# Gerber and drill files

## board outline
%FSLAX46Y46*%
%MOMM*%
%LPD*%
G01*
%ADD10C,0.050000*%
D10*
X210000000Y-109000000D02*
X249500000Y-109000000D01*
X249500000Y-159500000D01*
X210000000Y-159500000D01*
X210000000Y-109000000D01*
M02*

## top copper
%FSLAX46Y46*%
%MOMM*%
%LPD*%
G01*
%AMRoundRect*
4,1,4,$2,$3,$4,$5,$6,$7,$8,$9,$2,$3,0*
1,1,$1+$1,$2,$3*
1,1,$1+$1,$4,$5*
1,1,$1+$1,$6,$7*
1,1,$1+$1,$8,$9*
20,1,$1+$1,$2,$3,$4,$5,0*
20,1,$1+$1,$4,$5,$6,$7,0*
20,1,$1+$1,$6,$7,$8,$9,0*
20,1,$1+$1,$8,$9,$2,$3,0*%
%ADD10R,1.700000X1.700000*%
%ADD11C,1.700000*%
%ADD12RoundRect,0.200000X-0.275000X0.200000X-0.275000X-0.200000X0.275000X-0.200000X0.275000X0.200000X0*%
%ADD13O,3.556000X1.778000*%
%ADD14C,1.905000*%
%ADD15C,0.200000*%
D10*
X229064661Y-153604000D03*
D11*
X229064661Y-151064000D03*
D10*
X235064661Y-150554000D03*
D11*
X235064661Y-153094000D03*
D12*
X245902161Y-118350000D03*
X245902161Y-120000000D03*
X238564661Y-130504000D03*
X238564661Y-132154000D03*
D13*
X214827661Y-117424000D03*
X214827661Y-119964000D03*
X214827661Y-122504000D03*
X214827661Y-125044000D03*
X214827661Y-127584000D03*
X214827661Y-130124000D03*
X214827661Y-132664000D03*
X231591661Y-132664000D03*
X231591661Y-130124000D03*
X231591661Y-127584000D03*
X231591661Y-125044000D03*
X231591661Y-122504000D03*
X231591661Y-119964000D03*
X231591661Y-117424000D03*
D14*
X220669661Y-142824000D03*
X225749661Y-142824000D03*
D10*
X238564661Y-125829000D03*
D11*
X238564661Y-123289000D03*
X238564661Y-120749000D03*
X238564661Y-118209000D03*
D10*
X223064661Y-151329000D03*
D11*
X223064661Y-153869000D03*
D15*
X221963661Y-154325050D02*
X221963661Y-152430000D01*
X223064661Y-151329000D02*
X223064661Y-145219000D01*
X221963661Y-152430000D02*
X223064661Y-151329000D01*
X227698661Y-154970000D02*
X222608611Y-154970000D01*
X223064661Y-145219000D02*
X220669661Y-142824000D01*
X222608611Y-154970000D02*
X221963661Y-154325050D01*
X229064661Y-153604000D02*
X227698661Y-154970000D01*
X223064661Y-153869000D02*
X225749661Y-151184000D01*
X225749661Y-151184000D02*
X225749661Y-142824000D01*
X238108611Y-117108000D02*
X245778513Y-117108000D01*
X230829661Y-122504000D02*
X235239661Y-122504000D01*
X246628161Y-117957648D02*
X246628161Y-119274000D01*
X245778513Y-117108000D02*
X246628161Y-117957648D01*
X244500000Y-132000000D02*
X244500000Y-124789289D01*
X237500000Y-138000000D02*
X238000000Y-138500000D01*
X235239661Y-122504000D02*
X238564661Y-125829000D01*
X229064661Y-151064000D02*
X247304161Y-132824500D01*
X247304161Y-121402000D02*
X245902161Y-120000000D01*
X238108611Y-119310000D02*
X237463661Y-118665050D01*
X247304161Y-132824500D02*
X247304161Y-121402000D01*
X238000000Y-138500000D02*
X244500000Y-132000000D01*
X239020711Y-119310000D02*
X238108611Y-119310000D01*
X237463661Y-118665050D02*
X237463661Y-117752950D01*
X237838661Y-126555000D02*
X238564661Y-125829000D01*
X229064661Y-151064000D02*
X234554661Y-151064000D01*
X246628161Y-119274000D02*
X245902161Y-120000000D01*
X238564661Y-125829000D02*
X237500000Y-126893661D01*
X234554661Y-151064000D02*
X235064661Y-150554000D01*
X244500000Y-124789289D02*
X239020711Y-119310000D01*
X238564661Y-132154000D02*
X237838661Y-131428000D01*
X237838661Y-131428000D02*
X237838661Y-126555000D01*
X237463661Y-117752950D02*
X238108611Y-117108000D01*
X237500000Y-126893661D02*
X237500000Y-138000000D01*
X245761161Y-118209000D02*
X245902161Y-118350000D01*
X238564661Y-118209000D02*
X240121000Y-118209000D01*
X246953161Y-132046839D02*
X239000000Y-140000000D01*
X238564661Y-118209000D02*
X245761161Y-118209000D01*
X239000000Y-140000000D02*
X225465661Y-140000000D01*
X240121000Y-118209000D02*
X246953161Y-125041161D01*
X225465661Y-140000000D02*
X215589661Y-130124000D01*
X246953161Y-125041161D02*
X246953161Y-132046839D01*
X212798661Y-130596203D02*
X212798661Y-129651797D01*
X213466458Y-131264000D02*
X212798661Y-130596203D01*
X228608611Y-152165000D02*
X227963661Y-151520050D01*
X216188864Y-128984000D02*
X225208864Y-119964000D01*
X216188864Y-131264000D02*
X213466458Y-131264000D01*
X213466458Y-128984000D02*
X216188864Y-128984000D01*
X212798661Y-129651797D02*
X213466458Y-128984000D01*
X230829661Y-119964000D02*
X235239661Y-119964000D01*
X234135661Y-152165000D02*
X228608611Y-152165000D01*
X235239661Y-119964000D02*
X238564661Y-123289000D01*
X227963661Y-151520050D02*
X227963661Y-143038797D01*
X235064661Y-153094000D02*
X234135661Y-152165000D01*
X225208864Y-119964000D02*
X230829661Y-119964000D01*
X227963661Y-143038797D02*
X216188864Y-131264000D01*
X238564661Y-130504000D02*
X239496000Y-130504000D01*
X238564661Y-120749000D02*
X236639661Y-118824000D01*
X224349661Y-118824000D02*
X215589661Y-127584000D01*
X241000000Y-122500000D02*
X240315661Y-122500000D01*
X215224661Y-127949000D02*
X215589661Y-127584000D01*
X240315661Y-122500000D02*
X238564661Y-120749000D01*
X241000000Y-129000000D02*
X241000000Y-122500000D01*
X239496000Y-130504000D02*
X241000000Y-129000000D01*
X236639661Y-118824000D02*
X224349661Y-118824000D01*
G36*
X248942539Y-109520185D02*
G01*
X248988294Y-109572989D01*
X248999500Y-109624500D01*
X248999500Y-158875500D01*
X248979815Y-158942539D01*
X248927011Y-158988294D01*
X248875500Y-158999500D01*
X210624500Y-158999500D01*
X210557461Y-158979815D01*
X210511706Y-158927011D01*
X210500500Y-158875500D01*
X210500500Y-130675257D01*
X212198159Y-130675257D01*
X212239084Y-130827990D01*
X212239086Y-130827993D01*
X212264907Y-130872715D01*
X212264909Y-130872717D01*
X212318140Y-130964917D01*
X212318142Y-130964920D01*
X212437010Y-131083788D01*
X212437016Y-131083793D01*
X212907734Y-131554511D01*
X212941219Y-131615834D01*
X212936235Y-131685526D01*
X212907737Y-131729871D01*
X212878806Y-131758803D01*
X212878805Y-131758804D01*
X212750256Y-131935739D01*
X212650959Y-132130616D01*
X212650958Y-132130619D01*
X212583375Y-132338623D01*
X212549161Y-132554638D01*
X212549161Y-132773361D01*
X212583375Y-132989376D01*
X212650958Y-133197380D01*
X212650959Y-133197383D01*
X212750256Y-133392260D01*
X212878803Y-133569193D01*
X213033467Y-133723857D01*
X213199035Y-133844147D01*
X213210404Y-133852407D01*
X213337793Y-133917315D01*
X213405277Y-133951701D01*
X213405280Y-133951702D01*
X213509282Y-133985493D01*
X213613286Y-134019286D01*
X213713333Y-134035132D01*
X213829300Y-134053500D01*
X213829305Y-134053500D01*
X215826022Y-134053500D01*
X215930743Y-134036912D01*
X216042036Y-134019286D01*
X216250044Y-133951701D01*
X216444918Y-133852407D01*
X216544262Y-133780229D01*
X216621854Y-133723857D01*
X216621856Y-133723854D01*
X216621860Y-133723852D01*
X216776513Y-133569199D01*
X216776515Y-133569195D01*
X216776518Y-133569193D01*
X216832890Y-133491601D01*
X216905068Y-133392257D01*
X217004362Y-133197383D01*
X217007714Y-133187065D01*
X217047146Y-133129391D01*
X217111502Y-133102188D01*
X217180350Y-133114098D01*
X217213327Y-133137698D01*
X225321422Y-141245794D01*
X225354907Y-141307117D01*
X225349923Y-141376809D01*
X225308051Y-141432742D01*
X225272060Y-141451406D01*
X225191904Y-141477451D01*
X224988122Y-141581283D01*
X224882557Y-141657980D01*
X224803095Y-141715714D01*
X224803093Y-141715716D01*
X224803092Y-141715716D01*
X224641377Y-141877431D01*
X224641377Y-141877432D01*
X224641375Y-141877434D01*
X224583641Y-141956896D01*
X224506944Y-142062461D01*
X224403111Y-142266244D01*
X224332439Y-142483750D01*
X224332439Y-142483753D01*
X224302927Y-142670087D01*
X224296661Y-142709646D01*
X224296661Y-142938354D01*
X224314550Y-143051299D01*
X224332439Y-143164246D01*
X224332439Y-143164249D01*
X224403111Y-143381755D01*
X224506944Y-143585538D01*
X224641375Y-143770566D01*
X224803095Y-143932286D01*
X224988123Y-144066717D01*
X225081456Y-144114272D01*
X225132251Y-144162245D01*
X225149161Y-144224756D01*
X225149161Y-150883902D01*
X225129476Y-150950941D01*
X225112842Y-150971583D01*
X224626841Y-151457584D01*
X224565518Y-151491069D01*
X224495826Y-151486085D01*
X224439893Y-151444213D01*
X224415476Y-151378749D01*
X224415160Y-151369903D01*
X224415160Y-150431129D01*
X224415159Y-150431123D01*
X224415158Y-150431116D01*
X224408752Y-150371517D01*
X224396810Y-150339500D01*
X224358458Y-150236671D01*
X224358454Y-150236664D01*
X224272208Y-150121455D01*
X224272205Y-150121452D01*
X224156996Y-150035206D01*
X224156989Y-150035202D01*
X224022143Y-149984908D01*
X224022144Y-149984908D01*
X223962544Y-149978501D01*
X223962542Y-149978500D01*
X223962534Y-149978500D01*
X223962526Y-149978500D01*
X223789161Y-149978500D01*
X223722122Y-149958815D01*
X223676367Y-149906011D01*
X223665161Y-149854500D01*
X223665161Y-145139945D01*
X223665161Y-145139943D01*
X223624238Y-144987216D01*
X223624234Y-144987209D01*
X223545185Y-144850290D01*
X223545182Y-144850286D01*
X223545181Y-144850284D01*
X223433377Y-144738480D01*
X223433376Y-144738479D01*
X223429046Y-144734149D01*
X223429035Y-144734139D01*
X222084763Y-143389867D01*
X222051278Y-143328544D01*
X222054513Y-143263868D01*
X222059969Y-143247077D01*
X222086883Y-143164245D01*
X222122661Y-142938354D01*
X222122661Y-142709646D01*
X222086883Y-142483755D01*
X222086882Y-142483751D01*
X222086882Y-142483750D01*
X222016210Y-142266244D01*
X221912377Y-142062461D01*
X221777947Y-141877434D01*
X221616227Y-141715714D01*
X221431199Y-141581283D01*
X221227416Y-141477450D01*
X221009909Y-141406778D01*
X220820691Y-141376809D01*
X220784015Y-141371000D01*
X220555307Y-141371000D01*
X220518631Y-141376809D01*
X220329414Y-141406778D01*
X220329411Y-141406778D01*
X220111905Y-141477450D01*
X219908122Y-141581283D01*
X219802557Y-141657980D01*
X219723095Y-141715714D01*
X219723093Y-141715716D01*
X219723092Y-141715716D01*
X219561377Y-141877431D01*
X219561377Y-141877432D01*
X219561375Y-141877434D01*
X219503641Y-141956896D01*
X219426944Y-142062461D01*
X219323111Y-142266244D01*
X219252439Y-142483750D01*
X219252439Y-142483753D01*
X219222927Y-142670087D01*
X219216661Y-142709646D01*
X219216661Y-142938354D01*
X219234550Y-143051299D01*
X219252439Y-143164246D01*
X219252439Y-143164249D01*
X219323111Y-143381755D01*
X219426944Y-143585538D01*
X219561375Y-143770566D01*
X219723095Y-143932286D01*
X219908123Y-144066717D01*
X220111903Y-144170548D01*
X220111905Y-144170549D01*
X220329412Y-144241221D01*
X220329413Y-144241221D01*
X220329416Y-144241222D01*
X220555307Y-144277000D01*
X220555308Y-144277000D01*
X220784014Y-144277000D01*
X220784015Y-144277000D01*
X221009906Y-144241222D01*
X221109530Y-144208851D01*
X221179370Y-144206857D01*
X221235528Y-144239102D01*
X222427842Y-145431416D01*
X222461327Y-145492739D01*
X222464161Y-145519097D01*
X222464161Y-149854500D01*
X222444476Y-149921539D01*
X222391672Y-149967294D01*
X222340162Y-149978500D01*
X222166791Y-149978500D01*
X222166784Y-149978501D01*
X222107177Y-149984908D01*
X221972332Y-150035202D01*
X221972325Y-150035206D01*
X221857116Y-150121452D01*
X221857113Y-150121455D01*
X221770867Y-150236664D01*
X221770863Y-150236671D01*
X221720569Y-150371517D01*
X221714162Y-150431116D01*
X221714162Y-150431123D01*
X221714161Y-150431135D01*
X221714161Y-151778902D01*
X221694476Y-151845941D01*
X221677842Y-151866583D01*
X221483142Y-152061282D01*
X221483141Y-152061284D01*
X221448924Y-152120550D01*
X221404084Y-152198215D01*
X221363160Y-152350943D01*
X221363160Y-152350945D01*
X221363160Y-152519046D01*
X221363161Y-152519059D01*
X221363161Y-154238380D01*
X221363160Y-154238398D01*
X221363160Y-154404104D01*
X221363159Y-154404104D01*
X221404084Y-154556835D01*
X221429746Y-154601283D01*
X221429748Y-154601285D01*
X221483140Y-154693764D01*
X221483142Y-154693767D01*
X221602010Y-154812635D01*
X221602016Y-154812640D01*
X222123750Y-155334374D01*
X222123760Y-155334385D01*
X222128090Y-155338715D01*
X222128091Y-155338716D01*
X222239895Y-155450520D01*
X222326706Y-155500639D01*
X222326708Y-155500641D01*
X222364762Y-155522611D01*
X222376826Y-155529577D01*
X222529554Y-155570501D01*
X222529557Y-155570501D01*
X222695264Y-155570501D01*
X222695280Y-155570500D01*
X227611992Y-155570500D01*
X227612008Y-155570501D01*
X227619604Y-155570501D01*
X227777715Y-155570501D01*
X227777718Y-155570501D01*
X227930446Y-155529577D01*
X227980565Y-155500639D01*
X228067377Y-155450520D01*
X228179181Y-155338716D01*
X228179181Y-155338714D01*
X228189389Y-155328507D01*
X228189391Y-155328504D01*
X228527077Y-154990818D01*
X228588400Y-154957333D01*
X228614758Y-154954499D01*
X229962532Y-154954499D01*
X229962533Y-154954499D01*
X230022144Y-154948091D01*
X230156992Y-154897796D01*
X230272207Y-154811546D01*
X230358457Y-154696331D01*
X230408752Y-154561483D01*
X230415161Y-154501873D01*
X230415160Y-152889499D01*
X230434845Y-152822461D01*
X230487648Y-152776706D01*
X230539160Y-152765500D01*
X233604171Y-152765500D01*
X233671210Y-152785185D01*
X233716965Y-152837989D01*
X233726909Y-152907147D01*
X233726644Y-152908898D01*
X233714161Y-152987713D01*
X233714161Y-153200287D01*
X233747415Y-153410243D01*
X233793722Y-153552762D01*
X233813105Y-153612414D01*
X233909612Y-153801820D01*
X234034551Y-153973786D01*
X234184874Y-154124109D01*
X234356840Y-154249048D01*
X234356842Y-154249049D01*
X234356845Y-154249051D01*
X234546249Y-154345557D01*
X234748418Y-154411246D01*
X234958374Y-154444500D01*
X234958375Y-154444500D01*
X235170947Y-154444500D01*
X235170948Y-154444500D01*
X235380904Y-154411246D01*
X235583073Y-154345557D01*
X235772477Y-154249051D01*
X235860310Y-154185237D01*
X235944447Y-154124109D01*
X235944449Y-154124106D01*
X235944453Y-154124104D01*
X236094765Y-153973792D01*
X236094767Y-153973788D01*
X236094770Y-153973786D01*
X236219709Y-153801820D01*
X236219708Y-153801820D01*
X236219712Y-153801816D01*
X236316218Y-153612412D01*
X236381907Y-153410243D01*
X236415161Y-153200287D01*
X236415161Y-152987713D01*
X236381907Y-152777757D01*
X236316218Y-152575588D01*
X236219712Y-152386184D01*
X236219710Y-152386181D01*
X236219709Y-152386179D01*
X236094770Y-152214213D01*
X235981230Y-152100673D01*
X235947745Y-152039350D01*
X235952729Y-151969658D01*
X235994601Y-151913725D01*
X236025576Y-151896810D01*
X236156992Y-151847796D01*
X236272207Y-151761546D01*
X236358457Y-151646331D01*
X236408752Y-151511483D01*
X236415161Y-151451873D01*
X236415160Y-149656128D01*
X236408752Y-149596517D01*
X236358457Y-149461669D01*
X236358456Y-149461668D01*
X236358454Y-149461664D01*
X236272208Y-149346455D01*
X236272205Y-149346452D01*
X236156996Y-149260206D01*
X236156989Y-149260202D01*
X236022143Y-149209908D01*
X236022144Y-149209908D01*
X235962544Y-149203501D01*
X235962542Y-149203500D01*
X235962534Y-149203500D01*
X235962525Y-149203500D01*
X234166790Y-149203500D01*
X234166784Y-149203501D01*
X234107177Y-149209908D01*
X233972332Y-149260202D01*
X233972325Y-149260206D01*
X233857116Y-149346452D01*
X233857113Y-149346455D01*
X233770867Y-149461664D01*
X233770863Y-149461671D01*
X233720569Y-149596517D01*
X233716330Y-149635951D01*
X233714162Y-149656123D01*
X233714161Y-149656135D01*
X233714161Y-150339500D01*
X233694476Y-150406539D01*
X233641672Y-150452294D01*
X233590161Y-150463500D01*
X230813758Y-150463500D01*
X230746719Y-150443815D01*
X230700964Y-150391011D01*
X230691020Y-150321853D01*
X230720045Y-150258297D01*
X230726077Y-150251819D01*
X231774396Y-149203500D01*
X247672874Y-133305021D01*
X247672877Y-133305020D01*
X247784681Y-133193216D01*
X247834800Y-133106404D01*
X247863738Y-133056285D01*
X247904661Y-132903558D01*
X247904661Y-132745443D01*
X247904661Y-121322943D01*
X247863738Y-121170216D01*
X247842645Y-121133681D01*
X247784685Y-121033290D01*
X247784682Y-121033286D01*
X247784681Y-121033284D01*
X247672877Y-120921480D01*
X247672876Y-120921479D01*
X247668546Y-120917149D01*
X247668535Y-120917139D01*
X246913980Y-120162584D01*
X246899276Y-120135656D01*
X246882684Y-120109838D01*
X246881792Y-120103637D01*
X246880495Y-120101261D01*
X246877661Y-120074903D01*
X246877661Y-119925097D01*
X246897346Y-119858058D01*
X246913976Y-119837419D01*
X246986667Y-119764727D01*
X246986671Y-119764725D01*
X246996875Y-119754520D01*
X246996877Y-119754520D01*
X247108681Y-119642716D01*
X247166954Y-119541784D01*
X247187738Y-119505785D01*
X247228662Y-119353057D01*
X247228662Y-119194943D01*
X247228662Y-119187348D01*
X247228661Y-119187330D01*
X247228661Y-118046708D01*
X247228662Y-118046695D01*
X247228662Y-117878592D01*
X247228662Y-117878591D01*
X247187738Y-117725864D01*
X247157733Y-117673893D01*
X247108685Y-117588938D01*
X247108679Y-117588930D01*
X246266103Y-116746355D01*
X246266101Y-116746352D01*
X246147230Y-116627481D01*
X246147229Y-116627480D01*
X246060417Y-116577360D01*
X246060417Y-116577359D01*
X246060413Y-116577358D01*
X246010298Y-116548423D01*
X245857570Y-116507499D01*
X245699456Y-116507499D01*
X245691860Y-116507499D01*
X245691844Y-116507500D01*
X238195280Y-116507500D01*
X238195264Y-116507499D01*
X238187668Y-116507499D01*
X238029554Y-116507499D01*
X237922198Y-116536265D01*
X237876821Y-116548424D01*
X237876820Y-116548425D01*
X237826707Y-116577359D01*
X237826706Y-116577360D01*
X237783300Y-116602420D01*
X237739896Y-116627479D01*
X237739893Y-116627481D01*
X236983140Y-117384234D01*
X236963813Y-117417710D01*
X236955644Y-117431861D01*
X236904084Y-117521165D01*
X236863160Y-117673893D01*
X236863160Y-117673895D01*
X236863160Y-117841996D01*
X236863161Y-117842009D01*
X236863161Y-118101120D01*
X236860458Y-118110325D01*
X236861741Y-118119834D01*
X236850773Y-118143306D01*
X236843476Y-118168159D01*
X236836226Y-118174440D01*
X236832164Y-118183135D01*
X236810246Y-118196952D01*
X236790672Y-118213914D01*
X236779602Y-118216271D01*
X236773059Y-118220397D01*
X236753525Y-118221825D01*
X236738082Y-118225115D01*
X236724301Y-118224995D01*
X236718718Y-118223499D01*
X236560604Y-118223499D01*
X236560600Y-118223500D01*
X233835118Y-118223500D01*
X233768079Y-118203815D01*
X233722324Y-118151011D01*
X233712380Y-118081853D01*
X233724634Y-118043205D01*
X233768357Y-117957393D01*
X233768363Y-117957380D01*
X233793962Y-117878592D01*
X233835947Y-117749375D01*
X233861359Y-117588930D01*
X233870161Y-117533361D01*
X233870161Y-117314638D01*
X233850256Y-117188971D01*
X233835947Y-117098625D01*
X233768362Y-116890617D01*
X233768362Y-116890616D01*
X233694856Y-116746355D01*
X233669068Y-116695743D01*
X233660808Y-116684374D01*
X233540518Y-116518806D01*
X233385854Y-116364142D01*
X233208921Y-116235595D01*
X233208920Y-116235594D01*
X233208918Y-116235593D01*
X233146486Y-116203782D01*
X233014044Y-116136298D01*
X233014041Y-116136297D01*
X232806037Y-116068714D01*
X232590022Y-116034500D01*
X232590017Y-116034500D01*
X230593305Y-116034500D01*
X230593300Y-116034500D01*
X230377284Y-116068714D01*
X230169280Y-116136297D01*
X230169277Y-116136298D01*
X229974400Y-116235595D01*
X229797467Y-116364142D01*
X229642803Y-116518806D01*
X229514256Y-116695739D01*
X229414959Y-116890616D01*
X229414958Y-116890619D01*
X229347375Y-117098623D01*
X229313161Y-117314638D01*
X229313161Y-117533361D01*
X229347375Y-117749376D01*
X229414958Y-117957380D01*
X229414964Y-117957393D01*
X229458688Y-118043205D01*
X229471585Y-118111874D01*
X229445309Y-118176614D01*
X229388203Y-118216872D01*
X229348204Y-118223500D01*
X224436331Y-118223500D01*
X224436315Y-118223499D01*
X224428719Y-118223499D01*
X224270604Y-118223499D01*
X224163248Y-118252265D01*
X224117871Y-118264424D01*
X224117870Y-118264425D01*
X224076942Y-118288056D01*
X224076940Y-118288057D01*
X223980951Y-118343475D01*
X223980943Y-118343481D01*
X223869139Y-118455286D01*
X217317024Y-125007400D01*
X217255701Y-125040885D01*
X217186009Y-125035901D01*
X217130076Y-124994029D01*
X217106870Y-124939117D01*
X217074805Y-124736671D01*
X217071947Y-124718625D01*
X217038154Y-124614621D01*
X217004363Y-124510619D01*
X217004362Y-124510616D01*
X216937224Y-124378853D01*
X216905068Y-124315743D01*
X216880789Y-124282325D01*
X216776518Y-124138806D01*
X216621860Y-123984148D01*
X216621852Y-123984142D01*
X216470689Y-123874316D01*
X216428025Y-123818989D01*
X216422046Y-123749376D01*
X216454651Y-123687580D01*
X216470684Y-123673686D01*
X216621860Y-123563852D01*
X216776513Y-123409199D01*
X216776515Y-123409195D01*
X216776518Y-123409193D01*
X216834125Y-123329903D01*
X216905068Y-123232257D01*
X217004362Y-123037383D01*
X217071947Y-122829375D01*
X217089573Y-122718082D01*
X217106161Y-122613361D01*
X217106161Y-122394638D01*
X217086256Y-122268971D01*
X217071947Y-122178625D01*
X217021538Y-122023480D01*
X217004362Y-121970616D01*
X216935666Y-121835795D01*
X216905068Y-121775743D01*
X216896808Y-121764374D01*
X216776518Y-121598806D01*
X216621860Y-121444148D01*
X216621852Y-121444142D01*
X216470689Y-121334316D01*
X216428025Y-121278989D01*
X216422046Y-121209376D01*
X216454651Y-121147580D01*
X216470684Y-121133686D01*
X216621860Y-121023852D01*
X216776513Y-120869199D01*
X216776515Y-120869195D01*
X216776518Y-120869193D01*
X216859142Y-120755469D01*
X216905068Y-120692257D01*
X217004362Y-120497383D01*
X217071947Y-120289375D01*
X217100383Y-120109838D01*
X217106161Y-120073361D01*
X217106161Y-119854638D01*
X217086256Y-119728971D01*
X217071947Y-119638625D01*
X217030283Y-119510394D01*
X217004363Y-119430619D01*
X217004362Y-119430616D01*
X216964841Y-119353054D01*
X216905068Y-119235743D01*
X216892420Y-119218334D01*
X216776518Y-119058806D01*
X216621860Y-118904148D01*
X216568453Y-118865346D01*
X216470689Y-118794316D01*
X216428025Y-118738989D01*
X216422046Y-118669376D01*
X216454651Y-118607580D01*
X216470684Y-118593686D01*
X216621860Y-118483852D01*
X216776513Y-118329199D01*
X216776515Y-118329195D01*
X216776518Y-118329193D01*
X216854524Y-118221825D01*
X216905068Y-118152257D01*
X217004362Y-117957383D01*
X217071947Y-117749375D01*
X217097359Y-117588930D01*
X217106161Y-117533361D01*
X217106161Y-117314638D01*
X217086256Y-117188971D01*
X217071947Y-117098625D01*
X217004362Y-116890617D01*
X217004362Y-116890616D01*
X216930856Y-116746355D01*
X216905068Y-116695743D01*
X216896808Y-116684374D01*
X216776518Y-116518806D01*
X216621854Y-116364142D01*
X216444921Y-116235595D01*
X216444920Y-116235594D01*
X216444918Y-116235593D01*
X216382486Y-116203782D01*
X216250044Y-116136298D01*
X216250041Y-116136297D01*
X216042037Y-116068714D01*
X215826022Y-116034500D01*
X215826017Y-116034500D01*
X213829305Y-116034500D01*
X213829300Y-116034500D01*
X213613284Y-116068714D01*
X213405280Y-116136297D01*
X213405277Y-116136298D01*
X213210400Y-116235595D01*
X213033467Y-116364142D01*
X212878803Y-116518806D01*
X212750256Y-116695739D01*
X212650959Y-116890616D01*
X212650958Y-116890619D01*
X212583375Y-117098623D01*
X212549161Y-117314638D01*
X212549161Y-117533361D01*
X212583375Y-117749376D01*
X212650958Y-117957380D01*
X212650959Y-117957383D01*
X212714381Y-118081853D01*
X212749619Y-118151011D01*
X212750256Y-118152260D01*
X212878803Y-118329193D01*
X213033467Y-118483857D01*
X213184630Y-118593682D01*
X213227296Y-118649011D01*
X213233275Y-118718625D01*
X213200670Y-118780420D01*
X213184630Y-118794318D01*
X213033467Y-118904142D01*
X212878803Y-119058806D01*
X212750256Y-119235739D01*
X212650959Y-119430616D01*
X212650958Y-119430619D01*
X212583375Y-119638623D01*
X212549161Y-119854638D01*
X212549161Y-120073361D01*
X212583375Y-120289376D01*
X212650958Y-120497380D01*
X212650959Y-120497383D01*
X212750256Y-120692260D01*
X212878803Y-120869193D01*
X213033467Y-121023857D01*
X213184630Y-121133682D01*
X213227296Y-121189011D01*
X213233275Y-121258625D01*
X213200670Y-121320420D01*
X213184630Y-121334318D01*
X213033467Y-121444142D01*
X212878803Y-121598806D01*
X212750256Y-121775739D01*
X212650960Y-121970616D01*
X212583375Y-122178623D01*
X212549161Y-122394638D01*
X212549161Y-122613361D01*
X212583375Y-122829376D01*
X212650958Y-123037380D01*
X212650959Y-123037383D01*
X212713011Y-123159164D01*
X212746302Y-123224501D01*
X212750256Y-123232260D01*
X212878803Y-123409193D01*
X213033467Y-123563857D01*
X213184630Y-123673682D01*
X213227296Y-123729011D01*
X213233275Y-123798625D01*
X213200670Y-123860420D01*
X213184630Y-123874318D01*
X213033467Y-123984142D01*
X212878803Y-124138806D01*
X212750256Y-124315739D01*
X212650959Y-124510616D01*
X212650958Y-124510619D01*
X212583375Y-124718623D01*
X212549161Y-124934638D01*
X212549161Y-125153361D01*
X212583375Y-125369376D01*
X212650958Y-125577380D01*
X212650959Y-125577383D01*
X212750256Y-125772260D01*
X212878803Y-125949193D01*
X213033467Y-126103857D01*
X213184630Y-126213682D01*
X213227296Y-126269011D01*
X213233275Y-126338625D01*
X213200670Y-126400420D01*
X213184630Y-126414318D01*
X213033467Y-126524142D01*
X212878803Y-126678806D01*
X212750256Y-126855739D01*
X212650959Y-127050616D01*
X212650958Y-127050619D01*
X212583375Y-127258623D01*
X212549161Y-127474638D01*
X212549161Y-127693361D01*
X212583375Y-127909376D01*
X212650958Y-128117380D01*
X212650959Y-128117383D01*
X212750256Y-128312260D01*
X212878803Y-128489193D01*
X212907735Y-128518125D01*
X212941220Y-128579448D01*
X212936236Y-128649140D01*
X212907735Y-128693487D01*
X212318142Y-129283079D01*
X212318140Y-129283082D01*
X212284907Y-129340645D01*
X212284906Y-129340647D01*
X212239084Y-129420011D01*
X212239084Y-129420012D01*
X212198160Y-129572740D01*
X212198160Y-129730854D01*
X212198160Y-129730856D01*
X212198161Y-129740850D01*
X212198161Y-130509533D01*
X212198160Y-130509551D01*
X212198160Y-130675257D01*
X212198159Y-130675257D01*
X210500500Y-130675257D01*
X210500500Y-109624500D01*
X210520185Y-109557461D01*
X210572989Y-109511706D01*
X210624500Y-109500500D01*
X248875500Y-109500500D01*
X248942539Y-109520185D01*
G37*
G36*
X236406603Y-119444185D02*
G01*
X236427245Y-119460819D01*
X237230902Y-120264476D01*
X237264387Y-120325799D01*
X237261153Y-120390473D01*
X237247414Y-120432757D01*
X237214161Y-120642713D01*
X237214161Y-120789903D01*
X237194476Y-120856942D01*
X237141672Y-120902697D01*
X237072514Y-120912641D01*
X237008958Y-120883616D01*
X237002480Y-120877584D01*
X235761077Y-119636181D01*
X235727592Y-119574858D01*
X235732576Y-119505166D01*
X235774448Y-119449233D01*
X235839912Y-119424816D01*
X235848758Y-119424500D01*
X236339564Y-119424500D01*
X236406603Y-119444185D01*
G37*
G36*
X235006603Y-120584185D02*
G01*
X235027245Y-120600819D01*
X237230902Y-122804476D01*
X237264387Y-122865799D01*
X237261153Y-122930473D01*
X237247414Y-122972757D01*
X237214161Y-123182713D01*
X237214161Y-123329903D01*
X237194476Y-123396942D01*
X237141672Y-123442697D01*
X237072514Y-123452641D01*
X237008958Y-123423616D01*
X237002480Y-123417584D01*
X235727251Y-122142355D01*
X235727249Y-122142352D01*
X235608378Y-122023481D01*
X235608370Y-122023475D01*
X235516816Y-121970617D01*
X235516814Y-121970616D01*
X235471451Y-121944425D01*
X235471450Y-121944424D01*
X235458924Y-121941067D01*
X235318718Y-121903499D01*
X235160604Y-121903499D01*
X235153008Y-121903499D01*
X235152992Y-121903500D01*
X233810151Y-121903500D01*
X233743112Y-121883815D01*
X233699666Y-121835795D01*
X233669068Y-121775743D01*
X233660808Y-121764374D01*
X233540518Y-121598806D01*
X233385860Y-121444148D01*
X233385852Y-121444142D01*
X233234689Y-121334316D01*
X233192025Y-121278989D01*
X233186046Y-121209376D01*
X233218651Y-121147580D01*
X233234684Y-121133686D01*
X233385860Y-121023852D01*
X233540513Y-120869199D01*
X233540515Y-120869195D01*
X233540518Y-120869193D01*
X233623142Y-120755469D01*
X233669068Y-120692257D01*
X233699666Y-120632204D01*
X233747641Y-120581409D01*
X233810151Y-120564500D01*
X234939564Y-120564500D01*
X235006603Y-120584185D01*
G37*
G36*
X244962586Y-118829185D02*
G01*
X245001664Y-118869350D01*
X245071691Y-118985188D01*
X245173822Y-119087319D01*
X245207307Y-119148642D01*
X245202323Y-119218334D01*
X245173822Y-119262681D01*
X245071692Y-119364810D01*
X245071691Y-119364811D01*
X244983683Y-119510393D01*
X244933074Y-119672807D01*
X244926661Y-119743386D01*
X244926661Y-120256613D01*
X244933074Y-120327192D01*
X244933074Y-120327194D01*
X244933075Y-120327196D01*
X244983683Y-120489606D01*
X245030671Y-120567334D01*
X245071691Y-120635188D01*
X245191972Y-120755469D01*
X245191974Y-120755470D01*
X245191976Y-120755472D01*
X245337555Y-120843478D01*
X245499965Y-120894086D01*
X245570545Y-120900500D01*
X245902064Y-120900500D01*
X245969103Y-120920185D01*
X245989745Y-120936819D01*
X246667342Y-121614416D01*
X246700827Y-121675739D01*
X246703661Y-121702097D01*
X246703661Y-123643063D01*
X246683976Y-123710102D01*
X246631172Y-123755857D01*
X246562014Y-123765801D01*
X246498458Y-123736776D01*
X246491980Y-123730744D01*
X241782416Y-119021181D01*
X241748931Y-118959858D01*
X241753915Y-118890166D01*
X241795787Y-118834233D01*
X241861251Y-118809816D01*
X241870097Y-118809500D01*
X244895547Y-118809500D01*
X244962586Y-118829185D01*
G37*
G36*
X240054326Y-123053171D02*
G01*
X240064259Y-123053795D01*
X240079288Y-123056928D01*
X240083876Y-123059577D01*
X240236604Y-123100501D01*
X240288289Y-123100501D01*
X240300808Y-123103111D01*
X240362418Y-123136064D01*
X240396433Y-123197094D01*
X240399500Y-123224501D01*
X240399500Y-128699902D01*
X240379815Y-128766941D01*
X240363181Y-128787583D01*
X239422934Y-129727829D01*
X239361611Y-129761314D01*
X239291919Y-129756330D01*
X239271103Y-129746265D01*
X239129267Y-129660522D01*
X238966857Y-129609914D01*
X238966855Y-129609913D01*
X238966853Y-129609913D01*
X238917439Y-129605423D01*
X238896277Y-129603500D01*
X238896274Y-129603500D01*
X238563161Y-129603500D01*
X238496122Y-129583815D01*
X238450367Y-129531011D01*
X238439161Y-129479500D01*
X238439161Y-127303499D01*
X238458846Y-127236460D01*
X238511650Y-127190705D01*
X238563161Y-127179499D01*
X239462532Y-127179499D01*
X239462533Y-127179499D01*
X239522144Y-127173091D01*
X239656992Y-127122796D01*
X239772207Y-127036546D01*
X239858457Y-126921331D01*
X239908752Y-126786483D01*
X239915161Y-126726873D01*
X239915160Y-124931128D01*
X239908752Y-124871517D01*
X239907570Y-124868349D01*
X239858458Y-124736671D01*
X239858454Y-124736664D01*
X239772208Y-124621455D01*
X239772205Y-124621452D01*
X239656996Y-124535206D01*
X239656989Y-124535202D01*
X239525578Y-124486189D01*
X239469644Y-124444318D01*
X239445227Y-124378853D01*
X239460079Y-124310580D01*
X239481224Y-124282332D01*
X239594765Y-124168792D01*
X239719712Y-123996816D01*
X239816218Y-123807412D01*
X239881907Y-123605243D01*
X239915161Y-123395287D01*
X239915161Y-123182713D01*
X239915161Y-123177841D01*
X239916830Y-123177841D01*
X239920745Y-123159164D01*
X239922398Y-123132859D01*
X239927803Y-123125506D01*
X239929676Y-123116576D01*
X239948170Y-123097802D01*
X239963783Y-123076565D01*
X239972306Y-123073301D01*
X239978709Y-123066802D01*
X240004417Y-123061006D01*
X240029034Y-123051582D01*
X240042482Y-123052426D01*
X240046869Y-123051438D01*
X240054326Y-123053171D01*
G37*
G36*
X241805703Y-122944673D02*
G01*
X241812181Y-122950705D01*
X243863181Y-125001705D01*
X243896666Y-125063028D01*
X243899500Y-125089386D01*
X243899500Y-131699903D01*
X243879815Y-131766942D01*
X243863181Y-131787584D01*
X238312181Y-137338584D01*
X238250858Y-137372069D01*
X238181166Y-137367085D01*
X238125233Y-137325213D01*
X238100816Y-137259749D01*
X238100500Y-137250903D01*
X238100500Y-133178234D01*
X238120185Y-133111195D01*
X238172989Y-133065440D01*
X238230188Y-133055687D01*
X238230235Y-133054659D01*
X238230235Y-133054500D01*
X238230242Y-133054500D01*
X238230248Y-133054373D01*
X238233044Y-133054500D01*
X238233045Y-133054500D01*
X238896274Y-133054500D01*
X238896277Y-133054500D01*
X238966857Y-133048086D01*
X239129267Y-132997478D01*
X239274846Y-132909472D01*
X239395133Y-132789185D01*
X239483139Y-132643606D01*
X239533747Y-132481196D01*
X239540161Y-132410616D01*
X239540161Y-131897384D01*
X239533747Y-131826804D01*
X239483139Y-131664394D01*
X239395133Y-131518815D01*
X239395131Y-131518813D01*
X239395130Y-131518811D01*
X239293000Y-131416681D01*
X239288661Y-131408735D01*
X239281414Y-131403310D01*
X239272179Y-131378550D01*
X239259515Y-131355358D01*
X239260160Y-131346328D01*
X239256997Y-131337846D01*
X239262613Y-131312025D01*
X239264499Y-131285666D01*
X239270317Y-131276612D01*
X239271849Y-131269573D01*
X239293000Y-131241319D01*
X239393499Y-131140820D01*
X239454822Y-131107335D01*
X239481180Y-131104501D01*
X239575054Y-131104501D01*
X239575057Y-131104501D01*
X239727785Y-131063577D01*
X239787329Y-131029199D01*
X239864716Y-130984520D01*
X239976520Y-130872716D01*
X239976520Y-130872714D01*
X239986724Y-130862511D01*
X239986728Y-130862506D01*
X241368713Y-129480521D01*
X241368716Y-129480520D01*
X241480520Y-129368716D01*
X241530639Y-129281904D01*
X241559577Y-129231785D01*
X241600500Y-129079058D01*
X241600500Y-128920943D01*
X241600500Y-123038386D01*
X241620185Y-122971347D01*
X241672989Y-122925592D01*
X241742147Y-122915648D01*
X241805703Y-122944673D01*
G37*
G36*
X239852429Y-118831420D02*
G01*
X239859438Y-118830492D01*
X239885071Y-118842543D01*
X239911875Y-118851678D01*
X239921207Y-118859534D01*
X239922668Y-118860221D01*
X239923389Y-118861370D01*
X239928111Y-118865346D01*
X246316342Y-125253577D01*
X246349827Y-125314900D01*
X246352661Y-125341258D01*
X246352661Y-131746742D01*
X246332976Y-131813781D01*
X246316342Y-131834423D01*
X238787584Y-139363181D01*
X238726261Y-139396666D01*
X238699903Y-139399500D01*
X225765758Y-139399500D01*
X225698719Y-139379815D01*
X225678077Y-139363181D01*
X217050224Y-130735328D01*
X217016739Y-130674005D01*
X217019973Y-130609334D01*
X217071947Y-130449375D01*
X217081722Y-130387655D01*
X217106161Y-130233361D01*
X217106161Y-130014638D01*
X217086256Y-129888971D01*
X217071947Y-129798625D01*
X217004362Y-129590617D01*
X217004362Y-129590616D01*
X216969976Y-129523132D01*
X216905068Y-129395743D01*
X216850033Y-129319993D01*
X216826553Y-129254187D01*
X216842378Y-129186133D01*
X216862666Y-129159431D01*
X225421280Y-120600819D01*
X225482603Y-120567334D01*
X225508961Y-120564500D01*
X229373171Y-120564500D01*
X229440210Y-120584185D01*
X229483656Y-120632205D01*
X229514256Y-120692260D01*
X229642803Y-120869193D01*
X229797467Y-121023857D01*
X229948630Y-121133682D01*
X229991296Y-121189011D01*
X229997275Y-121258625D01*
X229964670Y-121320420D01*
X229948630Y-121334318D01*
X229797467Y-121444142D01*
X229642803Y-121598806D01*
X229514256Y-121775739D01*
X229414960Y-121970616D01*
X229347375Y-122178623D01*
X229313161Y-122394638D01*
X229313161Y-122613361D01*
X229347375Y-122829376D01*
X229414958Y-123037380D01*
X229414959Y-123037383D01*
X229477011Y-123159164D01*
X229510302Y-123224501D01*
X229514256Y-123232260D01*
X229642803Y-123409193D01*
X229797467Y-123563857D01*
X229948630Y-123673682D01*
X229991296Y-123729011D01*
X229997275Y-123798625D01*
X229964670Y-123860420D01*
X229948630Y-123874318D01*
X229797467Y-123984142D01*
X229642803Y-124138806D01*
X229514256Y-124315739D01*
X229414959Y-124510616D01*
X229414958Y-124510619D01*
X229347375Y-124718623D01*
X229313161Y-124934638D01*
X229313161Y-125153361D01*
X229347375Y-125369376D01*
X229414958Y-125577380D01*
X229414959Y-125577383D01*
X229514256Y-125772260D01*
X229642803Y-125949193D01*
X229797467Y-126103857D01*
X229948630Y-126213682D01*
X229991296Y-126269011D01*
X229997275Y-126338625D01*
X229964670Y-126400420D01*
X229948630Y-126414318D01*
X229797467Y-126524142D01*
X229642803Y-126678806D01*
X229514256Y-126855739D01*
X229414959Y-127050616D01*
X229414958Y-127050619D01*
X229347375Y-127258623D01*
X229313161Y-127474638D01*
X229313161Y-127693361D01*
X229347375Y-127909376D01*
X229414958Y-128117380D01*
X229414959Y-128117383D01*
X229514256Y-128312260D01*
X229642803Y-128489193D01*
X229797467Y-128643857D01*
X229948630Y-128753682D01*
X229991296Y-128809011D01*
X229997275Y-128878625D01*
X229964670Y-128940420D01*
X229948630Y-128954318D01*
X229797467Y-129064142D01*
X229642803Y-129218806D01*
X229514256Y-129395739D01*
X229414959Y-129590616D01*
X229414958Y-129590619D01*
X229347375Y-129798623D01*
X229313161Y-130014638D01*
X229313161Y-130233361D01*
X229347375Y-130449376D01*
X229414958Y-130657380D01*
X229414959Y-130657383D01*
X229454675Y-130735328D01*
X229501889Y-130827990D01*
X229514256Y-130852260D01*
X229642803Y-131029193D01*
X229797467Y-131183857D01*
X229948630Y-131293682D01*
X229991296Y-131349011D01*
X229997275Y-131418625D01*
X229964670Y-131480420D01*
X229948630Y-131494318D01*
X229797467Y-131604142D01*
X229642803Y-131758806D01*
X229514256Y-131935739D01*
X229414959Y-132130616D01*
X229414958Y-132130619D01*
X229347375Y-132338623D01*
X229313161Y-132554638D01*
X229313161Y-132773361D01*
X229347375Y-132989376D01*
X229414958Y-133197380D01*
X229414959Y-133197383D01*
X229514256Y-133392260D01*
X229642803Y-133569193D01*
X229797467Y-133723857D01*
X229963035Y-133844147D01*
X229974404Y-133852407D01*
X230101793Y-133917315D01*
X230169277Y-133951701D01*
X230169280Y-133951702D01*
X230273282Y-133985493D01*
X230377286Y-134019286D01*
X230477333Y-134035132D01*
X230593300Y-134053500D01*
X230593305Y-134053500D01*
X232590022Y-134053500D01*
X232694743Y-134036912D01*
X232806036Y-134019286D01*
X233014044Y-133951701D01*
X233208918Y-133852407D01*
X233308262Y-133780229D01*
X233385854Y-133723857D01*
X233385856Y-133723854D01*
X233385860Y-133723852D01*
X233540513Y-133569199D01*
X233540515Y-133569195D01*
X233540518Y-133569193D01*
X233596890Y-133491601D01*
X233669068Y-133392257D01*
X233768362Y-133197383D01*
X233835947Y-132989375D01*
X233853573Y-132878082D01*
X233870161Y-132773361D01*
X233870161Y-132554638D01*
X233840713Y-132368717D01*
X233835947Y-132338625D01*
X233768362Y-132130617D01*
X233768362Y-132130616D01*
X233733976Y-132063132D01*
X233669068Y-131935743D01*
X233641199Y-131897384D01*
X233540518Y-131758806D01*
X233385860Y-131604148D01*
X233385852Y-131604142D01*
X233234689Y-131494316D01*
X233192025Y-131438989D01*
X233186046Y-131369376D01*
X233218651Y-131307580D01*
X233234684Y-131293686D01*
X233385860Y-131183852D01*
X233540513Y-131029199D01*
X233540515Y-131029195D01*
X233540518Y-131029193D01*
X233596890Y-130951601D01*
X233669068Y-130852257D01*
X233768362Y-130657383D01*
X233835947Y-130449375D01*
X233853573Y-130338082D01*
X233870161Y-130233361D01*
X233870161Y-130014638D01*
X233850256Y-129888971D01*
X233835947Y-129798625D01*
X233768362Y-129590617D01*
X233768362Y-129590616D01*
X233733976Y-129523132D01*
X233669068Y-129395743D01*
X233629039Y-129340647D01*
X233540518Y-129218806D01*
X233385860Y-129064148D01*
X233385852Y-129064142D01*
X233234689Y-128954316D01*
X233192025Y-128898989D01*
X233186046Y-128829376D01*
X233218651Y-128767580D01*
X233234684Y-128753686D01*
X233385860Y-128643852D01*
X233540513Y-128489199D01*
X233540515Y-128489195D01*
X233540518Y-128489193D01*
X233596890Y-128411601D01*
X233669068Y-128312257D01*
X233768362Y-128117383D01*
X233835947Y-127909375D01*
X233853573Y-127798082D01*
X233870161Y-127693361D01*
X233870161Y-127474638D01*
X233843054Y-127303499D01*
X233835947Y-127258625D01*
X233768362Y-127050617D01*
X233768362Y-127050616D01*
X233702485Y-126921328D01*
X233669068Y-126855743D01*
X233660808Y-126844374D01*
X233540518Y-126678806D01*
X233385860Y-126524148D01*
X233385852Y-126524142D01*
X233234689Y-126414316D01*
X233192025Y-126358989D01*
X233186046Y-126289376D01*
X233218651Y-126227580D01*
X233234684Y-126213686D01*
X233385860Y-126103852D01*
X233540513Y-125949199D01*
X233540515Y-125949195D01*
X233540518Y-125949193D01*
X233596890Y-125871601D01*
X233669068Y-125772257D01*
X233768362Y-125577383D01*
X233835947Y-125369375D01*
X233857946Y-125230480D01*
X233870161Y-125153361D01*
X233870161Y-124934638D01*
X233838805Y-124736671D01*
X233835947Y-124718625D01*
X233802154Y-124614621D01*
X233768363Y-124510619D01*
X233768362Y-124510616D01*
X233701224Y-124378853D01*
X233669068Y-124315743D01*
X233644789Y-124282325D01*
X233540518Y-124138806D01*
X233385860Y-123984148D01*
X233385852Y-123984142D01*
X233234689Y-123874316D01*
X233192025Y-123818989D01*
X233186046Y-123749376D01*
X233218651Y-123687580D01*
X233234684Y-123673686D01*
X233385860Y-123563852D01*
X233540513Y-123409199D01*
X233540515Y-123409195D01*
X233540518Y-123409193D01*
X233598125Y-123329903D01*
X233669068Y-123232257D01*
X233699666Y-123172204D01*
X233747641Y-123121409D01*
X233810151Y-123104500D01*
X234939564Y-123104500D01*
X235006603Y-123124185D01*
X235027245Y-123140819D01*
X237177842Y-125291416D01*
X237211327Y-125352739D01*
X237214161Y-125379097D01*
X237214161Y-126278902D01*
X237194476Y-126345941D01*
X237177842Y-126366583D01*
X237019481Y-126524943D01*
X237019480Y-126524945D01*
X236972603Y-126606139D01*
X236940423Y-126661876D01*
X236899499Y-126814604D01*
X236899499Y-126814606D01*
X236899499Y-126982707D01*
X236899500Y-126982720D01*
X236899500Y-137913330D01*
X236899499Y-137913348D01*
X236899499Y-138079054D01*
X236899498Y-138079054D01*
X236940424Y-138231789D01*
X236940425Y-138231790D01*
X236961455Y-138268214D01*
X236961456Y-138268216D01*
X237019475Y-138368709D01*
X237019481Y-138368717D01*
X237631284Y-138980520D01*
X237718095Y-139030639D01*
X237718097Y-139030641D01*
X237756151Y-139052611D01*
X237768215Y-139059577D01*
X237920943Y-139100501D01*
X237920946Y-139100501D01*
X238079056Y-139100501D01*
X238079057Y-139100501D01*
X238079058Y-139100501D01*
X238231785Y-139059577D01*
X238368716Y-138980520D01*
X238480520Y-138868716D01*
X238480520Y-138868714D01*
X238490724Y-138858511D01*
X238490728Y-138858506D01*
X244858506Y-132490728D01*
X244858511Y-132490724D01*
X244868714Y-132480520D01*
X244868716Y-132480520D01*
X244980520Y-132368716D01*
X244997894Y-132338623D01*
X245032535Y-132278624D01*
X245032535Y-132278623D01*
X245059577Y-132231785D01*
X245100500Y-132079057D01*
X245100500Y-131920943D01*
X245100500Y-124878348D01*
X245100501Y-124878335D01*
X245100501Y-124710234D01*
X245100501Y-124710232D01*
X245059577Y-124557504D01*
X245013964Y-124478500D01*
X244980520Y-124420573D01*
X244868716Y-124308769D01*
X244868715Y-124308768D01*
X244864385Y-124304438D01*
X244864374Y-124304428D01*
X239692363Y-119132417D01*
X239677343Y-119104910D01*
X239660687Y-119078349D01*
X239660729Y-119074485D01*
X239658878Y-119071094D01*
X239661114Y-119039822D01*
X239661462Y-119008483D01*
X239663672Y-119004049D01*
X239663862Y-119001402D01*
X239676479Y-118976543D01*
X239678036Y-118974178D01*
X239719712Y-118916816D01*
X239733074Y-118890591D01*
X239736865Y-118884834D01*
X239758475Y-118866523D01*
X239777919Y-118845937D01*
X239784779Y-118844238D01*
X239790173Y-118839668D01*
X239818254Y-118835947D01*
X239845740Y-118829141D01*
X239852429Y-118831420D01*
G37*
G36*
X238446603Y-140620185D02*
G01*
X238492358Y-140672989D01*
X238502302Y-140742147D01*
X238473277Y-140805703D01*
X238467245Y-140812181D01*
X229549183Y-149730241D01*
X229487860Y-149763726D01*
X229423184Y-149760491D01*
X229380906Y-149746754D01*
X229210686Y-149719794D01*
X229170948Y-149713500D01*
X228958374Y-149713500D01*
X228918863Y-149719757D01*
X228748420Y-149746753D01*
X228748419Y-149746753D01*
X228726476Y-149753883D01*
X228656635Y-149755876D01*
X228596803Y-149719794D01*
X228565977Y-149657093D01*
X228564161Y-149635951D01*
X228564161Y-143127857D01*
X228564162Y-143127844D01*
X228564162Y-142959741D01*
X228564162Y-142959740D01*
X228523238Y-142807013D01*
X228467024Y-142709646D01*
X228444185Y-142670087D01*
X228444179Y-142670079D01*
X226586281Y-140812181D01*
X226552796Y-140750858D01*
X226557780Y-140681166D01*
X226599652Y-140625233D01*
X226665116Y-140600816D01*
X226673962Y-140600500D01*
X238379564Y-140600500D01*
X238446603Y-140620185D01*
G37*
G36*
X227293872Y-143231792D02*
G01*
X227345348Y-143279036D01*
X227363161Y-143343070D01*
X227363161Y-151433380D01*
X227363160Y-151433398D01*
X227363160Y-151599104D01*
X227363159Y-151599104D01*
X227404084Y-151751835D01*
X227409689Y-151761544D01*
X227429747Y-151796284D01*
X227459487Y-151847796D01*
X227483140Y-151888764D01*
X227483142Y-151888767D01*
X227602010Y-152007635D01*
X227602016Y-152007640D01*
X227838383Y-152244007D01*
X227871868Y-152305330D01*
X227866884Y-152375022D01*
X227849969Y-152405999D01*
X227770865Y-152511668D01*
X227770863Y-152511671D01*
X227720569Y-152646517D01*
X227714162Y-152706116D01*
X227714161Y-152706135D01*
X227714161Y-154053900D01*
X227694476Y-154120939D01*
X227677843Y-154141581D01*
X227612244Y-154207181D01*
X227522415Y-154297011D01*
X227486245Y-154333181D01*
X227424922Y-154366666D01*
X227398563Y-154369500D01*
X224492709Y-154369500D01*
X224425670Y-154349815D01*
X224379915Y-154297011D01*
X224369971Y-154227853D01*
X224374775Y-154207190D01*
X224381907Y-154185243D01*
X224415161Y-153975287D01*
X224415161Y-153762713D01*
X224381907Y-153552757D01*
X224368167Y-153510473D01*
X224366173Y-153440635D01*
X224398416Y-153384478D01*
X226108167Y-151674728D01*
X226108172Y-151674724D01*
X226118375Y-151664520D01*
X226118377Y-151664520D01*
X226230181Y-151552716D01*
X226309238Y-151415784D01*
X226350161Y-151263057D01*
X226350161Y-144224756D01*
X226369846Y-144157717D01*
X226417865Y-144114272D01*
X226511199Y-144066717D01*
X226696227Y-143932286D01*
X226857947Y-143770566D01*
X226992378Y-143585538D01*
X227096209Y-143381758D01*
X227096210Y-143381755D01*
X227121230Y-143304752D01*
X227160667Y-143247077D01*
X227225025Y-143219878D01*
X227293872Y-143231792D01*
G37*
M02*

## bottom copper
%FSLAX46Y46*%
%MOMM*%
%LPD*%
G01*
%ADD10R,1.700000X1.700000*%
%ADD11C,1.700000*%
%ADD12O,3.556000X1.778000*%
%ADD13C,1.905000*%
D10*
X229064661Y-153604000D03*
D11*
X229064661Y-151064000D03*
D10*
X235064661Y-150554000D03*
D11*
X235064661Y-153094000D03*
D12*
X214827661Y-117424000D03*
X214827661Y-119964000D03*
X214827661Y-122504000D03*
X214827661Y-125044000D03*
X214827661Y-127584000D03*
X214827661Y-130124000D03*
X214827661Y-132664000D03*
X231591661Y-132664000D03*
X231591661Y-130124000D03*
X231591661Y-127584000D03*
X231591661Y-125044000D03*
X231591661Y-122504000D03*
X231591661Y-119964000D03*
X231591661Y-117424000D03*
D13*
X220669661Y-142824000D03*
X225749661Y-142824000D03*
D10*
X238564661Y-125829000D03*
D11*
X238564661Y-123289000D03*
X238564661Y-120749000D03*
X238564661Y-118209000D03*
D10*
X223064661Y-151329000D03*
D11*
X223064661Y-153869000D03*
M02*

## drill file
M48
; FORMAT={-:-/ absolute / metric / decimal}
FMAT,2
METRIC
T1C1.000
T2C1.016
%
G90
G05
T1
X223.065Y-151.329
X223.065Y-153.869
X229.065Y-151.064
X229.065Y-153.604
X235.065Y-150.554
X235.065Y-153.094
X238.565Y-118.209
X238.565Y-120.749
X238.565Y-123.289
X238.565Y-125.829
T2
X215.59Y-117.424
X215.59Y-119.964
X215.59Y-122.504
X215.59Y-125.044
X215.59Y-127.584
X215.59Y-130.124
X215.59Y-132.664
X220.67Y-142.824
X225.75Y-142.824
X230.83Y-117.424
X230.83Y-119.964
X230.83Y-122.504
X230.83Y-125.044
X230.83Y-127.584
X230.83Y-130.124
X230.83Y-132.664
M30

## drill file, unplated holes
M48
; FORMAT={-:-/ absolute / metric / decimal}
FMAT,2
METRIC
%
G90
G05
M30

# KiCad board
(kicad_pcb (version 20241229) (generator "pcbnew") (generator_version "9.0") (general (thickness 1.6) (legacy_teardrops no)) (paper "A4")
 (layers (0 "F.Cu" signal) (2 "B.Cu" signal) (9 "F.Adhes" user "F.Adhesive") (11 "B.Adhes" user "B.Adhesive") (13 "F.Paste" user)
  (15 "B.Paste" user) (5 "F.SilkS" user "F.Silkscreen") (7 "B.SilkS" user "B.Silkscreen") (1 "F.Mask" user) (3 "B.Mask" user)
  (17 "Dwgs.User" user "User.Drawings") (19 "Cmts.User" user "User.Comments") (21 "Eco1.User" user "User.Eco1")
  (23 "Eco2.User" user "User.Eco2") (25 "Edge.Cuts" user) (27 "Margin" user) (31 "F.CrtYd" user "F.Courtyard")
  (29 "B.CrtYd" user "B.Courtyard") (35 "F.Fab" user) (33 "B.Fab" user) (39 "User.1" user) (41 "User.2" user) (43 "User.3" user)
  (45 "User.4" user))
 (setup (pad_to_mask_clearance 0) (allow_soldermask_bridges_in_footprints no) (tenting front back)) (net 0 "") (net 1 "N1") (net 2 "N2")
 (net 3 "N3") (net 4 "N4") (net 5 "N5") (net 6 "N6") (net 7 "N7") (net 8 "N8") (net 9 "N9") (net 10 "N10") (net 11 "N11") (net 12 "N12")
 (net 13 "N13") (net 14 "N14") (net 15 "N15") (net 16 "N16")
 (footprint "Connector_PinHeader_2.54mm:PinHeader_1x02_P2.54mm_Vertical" (layer "F.Cu") (at 229.064661 153.604 180)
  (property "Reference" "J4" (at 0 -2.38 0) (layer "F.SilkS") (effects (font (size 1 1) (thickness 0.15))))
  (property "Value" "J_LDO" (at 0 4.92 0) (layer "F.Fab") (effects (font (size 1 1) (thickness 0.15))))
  (pad "1" thru_hole rect (at 0 0 180) (size 1.7 1.7) (drill 1) (layers "*.Cu" "*.Mask") (remove_unused_layers no) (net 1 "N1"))
  (pad "2" thru_hole circle (at 0 2.54 180) (size 1.7 1.7) (drill 1) (layers "*.Cu" "*.Mask") (remove_unused_layers no) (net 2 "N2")))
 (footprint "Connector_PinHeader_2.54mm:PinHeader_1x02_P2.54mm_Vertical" (layer "F.Cu") (at 235.064661 150.554)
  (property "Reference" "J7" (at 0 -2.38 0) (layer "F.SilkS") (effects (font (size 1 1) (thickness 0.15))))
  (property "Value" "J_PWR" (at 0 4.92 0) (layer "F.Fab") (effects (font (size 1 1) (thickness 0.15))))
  (pad "1" thru_hole rect (at 0 0) (size 1.7 1.7) (drill 1) (layers "*.Cu" "*.Mask") (remove_unused_layers no) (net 2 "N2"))
  (pad "2" thru_hole circle (at 0 2.54) (size 1.7 1.7) (drill 1) (layers "*.Cu" "*.Mask") (remove_unused_layers no) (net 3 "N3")))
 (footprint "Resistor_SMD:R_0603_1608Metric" (layer "F.Cu") (at 245.902161 119.175 -90)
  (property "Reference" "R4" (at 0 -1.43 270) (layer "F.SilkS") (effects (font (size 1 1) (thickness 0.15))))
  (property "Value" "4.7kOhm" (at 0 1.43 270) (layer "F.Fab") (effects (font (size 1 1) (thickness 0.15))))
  (pad "1" smd roundrect (at -0.825 0 270) (size 0.8 0.95) (layers "F.Cu" "F.Mask" "F.Paste") (roundrect_rratio 0.25) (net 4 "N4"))
  (pad "2" smd roundrect (at 0.825 0 270) (size 0.8 0.95) (layers "F.Cu" "F.Mask" "F.Paste") (roundrect_rratio 0.25) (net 2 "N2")))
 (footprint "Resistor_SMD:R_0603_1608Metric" (layer "F.Cu") (at 238.564661 131.329 -90)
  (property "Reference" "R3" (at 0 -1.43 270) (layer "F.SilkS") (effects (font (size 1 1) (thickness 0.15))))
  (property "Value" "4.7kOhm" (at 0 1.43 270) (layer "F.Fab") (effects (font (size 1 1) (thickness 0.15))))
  (pad "1" smd roundrect (at -0.825 0 270) (size 0.8 0.95) (layers "F.Cu" "F.Mask" "F.Paste") (roundrect_rratio 0.25) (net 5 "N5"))
  (pad "2" smd roundrect (at 0.825 0 270) (size 0.8 0.95) (layers "F.Cu" "F.Mask" "F.Paste") (roundrect_rratio 0.25) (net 2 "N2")))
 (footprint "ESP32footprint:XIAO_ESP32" (layer "F.Cu") (at 223.209661 125.044)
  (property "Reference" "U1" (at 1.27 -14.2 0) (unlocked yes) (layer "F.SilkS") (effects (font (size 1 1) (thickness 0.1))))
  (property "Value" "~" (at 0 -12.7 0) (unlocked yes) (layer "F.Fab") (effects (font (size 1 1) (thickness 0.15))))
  (pad "1" thru_hole oval (at -7.62 -7.62) (size 3.556 1.778) (drill 1.016 (offset -0.762 0)) (layers "*.Cu" "*.Mask")
   (remove_unused_layers no) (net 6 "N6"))
  (pad "2" thru_hole oval (at -7.62 -5.08) (size 3.556 1.778) (drill 1.016 (offset -0.762 0)) (layers "*.Cu" "*.Mask")
   (remove_unused_layers no) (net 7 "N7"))
  (pad "3" thru_hole oval (at -7.62 -2.54) (size 3.556 1.778) (drill 1.016 (offset -0.762 0)) (layers "*.Cu" "*.Mask")
   (remove_unused_layers no) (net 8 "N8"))
  (pad "4" thru_hole oval (at -7.62 0) (size 3.556 1.778) (drill 1.016 (offset -0.762 0)) (layers "*.Cu" "*.Mask") (remove_unused_layers no)
   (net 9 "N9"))
  (pad "5" thru_hole oval (at -7.62 2.54) (size 3.556 1.778) (drill 1.016 (offset -0.762 0)) (layers "*.Cu" "*.Mask")
   (remove_unused_layers no) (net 5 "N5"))
  (pad "6" thru_hole oval (at -7.62 5.08) (size 3.556 1.778) (drill 1.016 (offset -0.762 0)) (layers "*.Cu" "*.Mask")
   (remove_unused_layers no) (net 4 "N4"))
  (pad "7" thru_hole oval (at -7.62 7.62) (size 3.556 1.778) (drill 1.016 (offset -0.762 0)) (layers "*.Cu" "*.Mask")
   (remove_unused_layers no) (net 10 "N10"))
  (pad "8" thru_hole oval (at 7.62 7.62) (size 3.556 1.778) (drill 1.016 (offset 0.762 0)) (layers "*.Cu" "*.Mask")
   (remove_unused_layers no) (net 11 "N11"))
  (pad "9" thru_hole oval (at 7.62 5.08) (size 3.556 1.778) (drill 1.016 (offset 0.762 0)) (layers "*.Cu" "*.Mask")
   (remove_unused_layers no) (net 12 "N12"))
  (pad "10" thru_hole oval (at 7.62 2.54) (size 3.556 1.778) (drill 1.016 (offset 0.762 0)) (layers "*.Cu" "*.Mask")
   (remove_unused_layers no) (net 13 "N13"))
  (pad "11" thru_hole oval (at 7.62 0) (size 3.556 1.778) (drill 1.016 (offset 0.762 0)) (layers "*.Cu" "*.Mask") (remove_unused_layers no)
   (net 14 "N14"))
  (pad "12" thru_hole oval (at 7.62 -2.54) (size 3.556 1.778) (drill 1.016 (offset 0.762 0)) (layers "*.Cu" "*.Mask")
   (remove_unused_layers no) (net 2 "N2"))
  (pad "13" thru_hole oval (at 7.62 -5.08) (size 3.556 1.778) (drill 1.016 (offset 0.762 0)) (layers "*.Cu" "*.Mask")
   (remove_unused_layers no) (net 3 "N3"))
  (pad "14" thru_hole oval (at 7.62 -7.62) (size 3.556 1.778) (drill 1.016 (offset 0.762 0)) (layers "*.Cu" "*.Mask")
   (remove_unused_layers no) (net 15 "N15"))
  (pad "15" thru_hole circle (at -2.54 17.78) (size 1.905 1.905) (drill 1.016) (layers "*.Cu" "*.Mask") (remove_unused_layers no)
   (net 1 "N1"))
  (pad "16" thru_hole circle (at 2.54 17.78) (size 1.905 1.905) (drill 1.016) (layers "*.Cu" "*.Mask") (remove_unused_layers no)
   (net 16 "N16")))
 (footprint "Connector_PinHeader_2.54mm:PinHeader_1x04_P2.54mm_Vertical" (layer "F.Cu") (at 238.564661 125.829 180)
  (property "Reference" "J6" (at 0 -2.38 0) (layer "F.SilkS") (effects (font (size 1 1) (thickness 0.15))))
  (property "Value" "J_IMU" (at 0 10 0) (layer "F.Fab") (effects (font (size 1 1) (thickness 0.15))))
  (pad "1" thru_hole rect (at 0 0 180) (size 1.7 1.7) (drill 1) (layers "*.Cu" "*.Mask") (remove_unused_layers no) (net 2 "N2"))
  (pad "2" thru_hole circle (at 0 2.54 180) (size 1.7 1.7) (drill 1) (layers "*.Cu" "*.Mask") (remove_unused_layers no) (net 3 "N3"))
  (pad "3" thru_hole circle (at 0 5.08 180) (size 1.7 1.7) (drill 1) (layers "*.Cu" "*.Mask") (remove_unused_layers no) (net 5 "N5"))
  (pad "4" thru_hole circle (at 0 7.62 180) (size 1.7 1.7) (drill 1) (layers "*.Cu" "*.Mask") (remove_unused_layers no) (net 4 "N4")))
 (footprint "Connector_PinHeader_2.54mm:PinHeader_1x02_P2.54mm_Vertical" (layer "F.Cu") (at 223.064661 151.329)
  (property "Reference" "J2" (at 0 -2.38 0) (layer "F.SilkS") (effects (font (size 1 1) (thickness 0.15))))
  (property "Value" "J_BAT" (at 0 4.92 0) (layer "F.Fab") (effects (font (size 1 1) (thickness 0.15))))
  (pad "1" thru_hole rect (at 0 0) (size 1.7 1.7) (drill 1) (layers "*.Cu" "*.Mask") (remove_unused_layers no) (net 1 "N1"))
  (pad "2" thru_hole circle (at 0 2.54) (size 1.7 1.7) (drill 1) (layers "*.Cu" "*.Mask") (remove_unused_layers no) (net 16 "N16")))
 (gr_rect (start 210 109) (end 249.5 159.5) (stroke (width 0.05) (type default)) (fill no) (layer "Edge.Cuts"))
 (segment (start 221.963661 154.32505) (end 221.963661 152.43) (width 0.2) (layer "F.Cu") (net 1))
 (segment (start 223.064661 151.329) (end 223.064661 145.219) (width 0.2) (layer "F.Cu") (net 1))
 (segment (start 221.963661 152.43) (end 223.064661 151.329) (width 0.2) (layer "F.Cu") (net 1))
 (segment (start 227.698661 154.97) (end 222.608611 154.97) (width 0.2) (layer "F.Cu") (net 1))
 (segment (start 223.064661 145.219) (end 220.669661 142.824) (width 0.2) (layer "F.Cu") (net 1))
 (segment (start 222.608611 154.97) (end 221.963661 154.32505) (width 0.2) (layer "F.Cu") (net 1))
 (segment (start 229.064661 153.604) (end 227.698661 154.97) (width 0.2) (layer "F.Cu") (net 1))
 (segment (start 223.064661 153.869) (end 225.749661 151.184) (width 0.2) (layer "F.Cu") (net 16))
 (segment (start 225.749661 151.184) (end 225.749661 142.824) (width 0.2) (layer "F.Cu") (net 16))
 (segment (start 238.108611 117.108) (end 245.778513 117.108) (width 0.2) (layer "F.Cu") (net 2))
 (segment (start 230.829661 122.504) (end 235.239661 122.504) (width 0.2) (layer "F.Cu") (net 2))
 (segment (start 246.628161 117.957648) (end 246.628161 119.274) (width 0.2) (layer "F.Cu") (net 2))
 (segment (start 245.778513 117.108) (end 246.628161 117.957648) (width 0.2) (layer "F.Cu") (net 2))
 (segment (start 244.5 132) (end 244.5 124.789289) (width 0.2) (layer "F.Cu") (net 2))
 (segment (start 237.5 138) (end 238 138.5) (width 0.2) (layer "F.Cu") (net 2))
 (segment (start 235.239661 122.504) (end 238.564661 125.829) (width 0.2) (layer "F.Cu") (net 2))
 (segment (start 229.064661 151.064) (end 247.304161 132.8245) (width 0.2) (layer "F.Cu") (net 2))
 (segment (start 247.304161 121.402) (end 245.902161 120) (width 0.2) (layer "F.Cu") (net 2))
 (segment (start 238.108611 119.31) (end 237.463661 118.66505) (width 0.2) (layer "F.Cu") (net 2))
 (segment (start 247.304161 132.8245) (end 247.304161 121.402) (width 0.2) (layer "F.Cu") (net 2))
 (segment (start 238 138.5) (end 244.5 132) (width 0.2) (layer "F.Cu") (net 2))
 (segment (start 239.020711 119.31) (end 238.108611 119.31) (width 0.2) (layer "F.Cu") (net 2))
 (segment (start 237.463661 118.66505) (end 237.463661 117.75295) (width 0.2) (layer "F.Cu") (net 2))
 (segment (start 237.838661 126.555) (end 238.564661 125.829) (width 0.2) (layer "F.Cu") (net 2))
 (segment (start 229.064661 151.064) (end 234.554661 151.064) (width 0.2) (layer "F.Cu") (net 2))
 (segment (start 246.628161 119.274) (end 245.902161 120) (width 0.2) (layer "F.Cu") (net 2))
 (segment (start 238.564661 125.829) (end 237.5 126.893661) (width 0.2) (layer "F.Cu") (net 2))
 (segment (start 234.554661 151.064) (end 235.064661 150.554) (width 0.2) (layer "F.Cu") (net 2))
 (segment (start 244.5 124.789289) (end 239.020711 119.31) (width 0.2) (layer "F.Cu") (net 2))
 (segment (start 238.564661 132.154) (end 237.838661 131.428) (width 0.2) (layer "F.Cu") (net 2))
 (segment (start 237.838661 131.428) (end 237.838661 126.555) (width 0.2) (layer "F.Cu") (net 2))
 (segment (start 237.463661 117.75295) (end 238.108611 117.108) (width 0.2) (layer "F.Cu") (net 2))
 (segment (start 237.5 126.893661) (end 237.5 138) (width 0.2) (layer "F.Cu") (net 2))
 (segment (start 245.761161 118.209) (end 245.902161 118.35) (width 0.2) (layer "F.Cu") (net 4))
 (segment (start 238.564661 118.209) (end 240.121 118.209) (width 0.2) (layer "F.Cu") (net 4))
 (segment (start 246.953161 132.046839) (end 239 140) (width 0.2) (layer "F.Cu") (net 4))
 (segment (start 238.564661 118.209) (end 245.761161 118.209) (width 0.2) (layer "F.Cu") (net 4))
 (segment (start 239 140) (end 225.465661 140) (width 0.2) (layer "F.Cu") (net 4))
 (segment (start 240.121 118.209) (end 246.953161 125.041161) (width 0.2) (layer "F.Cu") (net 4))
 (segment (start 225.465661 140) (end 215.589661 130.124) (width 0.2) (layer "F.Cu") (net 4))
 (segment (start 246.953161 125.041161) (end 246.953161 132.046839) (width 0.2) (layer "F.Cu") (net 4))
 (segment (start 212.798661 130.596203) (end 212.798661 129.651797) (width 0.2) (layer "F.Cu") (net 3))
 (segment (start 213.466458 131.264) (end 212.798661 130.596203) (width 0.2) (layer "F.Cu") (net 3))
 (segment (start 228.608611 152.165) (end 227.963661 151.52005) (width 0.2) (layer "F.Cu") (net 3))
 (segment (start 216.188864 128.984) (end 225.208864 119.964) (width 0.2) (layer "F.Cu") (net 3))
 (segment (start 216.188864 131.264) (end 213.466458 131.264) (width 0.2) (layer "F.Cu") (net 3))
 (segment (start 213.466458 128.984) (end 216.188864 128.984) (width 0.2) (layer "F.Cu") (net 3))
 (segment (start 212.798661 129.651797) (end 213.466458 128.984) (width 0.2) (layer "F.Cu") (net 3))
 (segment (start 230.829661 119.964) (end 235.239661 119.964) (width 0.2) (layer "F.Cu") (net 3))
 (segment (start 234.135661 152.165) (end 228.608611 152.165) (width 0.2) (layer "F.Cu") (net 3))
 (segment (start 235.239661 119.964) (end 238.564661 123.289) (width 0.2) (layer "F.Cu") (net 3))
 (segment (start 227.963661 151.52005) (end 227.963661 143.038797) (width 0.2) (layer "F.Cu") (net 3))
 (segment (start 235.064661 153.094) (end 234.135661 152.165) (width 0.2) (layer "F.Cu") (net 3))
 (segment (start 225.208864 119.964) (end 230.829661 119.964) (width 0.2) (layer "F.Cu") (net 3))
 (segment (start 227.963661 143.038797) (end 216.188864 131.264) (width 0.2) (layer "F.Cu") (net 3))
 (segment (start 238.564661 130.504) (end 239.496 130.504) (width 0.2) (layer "F.Cu") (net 5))
 (segment (start 238.564661 120.749) (end 236.639661 118.824) (width 0.2) (layer "F.Cu") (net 5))
 (segment (start 224.349661 118.824) (end 215.589661 127.584) (width 0.2) (layer "F.Cu") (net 5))
 (segment (start 241 122.5) (end 240.315661 122.5) (width 0.2) (layer "F.Cu") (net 5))
 (segment (start 215.224661 127.949) (end 215.589661 127.584) (width 0.2) (layer "F.Cu") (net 5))
 (segment (start 240.315661 122.5) (end 238.564661 120.749) (width 0.2) (layer "F.Cu") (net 5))
 (segment (start 241 129) (end 241 122.5) (width 0.2) (layer "F.Cu") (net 5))
 (segment (start 239.496 130.504) (end 241 129) (width 0.2) (layer "F.Cu") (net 5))
 (segment (start 236.639661 118.824) (end 224.349661 118.824) (width 0.2) (layer "F.Cu") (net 5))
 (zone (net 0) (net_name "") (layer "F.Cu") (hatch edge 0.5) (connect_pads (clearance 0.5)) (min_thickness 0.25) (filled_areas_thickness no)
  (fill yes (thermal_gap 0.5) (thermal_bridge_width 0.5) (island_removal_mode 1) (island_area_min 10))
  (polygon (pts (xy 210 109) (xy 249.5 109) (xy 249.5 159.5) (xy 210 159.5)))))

